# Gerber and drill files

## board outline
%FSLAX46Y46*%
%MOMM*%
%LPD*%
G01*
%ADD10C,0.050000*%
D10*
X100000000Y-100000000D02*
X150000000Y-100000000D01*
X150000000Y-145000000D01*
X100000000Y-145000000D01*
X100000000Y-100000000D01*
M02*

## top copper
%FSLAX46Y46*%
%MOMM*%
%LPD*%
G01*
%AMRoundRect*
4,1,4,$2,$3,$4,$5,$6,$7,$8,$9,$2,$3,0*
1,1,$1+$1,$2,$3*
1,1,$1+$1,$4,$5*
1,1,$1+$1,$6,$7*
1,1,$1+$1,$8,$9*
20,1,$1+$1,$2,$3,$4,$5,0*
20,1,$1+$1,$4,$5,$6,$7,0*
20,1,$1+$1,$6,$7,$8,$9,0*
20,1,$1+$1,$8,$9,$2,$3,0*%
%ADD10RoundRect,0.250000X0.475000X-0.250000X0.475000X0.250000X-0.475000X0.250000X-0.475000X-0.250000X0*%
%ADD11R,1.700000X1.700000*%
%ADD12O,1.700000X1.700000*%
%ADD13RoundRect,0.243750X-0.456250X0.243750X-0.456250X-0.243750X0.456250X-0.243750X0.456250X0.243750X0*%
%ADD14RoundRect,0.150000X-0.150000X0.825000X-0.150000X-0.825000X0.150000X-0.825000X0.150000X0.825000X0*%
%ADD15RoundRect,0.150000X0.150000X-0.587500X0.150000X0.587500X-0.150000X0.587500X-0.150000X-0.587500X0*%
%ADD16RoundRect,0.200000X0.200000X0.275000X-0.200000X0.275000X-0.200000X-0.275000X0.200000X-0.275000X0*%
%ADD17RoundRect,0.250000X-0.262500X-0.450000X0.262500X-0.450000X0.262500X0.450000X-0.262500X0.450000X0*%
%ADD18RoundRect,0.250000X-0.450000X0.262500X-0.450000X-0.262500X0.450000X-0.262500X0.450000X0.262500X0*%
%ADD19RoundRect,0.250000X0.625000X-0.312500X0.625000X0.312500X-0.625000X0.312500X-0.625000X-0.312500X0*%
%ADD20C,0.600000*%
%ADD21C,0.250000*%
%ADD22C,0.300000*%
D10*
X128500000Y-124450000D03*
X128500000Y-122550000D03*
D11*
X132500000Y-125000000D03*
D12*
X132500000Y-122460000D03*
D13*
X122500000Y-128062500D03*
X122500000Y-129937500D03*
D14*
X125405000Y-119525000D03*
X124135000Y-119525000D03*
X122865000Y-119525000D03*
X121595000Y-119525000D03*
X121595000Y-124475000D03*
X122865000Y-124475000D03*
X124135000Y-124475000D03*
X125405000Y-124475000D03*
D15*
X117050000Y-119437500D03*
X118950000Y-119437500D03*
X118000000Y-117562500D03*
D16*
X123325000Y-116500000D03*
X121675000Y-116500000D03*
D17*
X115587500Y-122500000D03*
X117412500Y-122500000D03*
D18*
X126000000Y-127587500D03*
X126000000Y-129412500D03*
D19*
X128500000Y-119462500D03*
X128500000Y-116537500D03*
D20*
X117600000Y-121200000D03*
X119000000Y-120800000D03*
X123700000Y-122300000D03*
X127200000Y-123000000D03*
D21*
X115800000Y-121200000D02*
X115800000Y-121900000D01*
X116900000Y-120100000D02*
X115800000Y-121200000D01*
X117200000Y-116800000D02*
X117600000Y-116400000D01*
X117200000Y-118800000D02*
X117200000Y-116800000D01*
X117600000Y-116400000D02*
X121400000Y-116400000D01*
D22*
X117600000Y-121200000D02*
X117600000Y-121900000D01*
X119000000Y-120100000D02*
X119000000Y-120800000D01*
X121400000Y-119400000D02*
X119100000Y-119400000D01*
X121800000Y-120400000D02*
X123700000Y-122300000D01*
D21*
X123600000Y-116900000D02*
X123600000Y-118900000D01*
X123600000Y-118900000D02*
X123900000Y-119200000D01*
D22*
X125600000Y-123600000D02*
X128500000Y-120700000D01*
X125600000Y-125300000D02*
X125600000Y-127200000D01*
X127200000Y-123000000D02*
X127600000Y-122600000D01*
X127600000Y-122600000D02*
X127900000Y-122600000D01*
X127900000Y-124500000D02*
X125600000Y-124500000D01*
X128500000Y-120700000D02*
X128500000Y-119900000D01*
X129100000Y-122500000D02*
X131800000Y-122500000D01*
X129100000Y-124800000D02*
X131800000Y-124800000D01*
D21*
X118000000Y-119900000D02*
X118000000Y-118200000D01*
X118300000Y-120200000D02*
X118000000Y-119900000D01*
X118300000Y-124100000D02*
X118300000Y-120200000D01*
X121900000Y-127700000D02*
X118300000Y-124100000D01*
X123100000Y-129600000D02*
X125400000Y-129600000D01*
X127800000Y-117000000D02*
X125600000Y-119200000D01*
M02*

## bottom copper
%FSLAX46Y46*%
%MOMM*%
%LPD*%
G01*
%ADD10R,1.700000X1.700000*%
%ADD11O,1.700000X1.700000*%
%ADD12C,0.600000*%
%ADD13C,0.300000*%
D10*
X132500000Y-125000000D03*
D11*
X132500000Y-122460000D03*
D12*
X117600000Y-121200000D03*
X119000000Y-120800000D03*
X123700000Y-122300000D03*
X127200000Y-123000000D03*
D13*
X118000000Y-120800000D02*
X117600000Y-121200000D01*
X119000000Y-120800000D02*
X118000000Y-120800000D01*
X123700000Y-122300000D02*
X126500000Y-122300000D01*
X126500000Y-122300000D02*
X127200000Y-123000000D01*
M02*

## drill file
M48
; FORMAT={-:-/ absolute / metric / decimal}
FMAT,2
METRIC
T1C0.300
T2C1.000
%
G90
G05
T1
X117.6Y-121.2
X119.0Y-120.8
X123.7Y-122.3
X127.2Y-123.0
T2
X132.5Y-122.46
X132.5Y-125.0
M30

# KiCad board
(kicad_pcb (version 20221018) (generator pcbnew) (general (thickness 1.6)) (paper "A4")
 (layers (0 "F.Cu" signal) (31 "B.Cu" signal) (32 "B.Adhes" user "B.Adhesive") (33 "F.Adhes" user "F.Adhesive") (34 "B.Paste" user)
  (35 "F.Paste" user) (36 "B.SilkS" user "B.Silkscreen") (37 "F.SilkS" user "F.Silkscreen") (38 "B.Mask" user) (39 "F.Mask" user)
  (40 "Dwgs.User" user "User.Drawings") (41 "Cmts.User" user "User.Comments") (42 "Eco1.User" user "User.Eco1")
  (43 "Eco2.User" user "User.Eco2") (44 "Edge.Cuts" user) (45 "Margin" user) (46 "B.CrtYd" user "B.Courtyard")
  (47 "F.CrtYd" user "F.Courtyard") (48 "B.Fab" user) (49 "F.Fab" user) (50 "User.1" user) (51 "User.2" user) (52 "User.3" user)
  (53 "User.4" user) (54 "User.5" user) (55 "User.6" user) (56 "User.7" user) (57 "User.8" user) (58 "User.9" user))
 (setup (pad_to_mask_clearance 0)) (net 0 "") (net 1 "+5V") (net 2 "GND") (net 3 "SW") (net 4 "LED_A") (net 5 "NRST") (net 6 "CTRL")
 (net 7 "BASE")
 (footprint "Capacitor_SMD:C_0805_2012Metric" (layer "F.Cu") (at 128.5 123.5 90)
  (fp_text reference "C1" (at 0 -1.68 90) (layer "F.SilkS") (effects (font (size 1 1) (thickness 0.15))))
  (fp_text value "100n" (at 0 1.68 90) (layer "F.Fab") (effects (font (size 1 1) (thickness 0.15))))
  (pad "1" smd roundrect (at -0.95 0 90) (size 1 1.45) (layers "F.Cu" "F.Paste" "F.Mask") (roundrect_rratio 0.25) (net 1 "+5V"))
  (pad "2" smd roundrect (at 0.95 0 90) (size 1 1.45) (layers "F.Cu" "F.Paste" "F.Mask") (roundrect_rratio 0.25) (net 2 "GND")))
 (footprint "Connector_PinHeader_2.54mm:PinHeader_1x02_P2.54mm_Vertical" (layer "F.Cu") (at 132.5 125 180)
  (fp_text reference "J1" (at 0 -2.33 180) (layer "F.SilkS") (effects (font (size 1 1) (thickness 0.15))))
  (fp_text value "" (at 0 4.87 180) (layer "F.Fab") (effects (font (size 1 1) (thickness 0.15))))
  (pad "1" thru_hole rect (at 0 0 180) (size 1.7 1.7) (drill 1) (layers "*.Cu" "*.Mask") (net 1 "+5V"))
  (pad "2" thru_hole oval (at 0 2.54 180) (size 1.7 1.7) (drill 1) (layers "*.Cu" "*.Mask") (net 2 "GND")))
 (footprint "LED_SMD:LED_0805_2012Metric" (layer "F.Cu") (at 122.5 129 -90)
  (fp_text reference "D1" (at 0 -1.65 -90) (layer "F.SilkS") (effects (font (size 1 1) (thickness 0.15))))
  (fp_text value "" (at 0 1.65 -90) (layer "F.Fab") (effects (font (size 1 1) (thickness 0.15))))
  (pad "1" smd roundrect (at -0.9375 0 270) (size 0.975 1.4) (layers "F.Cu" "F.Paste" "F.Mask") (roundrect_rratio 0.25) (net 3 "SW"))
  (pad "2" smd roundrect (at 0.9375 0 270) (size 0.975 1.4) (layers "F.Cu" "F.Paste" "F.Mask") (roundrect_rratio 0.25) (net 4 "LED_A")))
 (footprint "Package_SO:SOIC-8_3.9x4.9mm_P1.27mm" (layer "F.Cu") (at 123.5 122 -90)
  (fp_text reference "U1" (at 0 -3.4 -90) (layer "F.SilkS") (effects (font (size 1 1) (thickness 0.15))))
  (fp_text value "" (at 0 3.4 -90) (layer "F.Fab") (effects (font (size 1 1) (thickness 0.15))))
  (pad "1" smd roundrect (at -2.475 -1.905 270) (size 1.95 0.6) (layers "F.Cu" "F.Paste" "F.Mask") (roundrect_rratio 0.25) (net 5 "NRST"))
  (pad "2" smd roundrect (at -2.475 -0.635 270) (size 1.95 0.6) (layers "F.Cu" "F.Paste" "F.Mask") (roundrect_rratio 0.25) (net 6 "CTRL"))
  (pad "3" smd roundrect (at -2.475 0.635 270) (size 1.95 0.6) (layers "F.Cu" "F.Paste" "F.Mask") (roundrect_rratio 0.25))
  (pad "4" smd roundrect (at -2.475 1.905 270) (size 1.95 0.6) (layers "F.Cu" "F.Paste" "F.Mask") (roundrect_rratio 0.25) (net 2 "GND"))
  (pad "5" smd roundrect (at 2.475 1.905 270) (size 1.95 0.6) (layers "F.Cu" "F.Paste" "F.Mask") (roundrect_rratio 0.25))
  (pad "6" smd roundrect (at 2.475 0.635 270) (size 1.95 0.6) (layers "F.Cu" "F.Paste" "F.Mask") (roundrect_rratio 0.25))
  (pad "7" smd roundrect (at 2.475 -0.635 270) (size 1.95 0.6) (layers "F.Cu" "F.Paste" "F.Mask") (roundrect_rratio 0.25))
  (pad "8" smd roundrect (at 2.475 -1.905 270) (size 1.95 0.6) (layers "F.Cu" "F.Paste" "F.Mask") (roundrect_rratio 0.25) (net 1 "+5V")))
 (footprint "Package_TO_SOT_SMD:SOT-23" (layer "F.Cu") (at 118 118.5 90)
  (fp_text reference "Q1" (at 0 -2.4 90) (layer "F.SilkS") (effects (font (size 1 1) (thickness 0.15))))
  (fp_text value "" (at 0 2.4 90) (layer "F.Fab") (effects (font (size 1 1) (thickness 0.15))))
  (pad "1" smd roundrect (at -0.9375 -0.95 90) (size 1.475 0.6) (layers "F.Cu" "F.Paste" "F.Mask") (roundrect_rratio 0.25) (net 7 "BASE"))
  (pad "2" smd roundrect (at -0.9375 0.95 90) (size 1.475 0.6) (layers "F.Cu" "F.Paste" "F.Mask") (roundrect_rratio 0.25) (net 2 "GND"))
  (pad "3" smd roundrect (at 0.9375 0 90) (size 1.475 0.6) (layers "F.Cu" "F.Paste" "F.Mask") (roundrect_rratio 0.25) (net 3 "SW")))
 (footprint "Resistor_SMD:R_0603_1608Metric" (layer "F.Cu") (at 122.5 116.5 180)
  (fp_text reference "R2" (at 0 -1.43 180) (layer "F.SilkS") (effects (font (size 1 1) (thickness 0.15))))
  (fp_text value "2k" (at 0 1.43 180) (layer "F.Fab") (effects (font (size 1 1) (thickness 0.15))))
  (pad "1" smd roundrect (at -0.825 0 180) (size 0.8 0.95) (layers "F.Cu" "F.Paste" "F.Mask") (roundrect_rratio 0.25) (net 6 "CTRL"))
  (pad "2" smd roundrect (at 0.825 0 180) (size 0.8 0.95) (layers "F.Cu" "F.Paste" "F.Mask") (roundrect_rratio 0.25) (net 7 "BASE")))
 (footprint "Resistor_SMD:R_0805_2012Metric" (layer "F.Cu") (at 116.5 122.5)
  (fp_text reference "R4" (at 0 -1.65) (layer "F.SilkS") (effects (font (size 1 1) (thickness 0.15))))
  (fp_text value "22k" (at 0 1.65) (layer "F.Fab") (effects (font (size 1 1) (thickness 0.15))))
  (pad "1" smd roundrect (at -0.9125 0) (size 1.025 1.4) (layers "F.Cu" "F.Paste" "F.Mask") (roundrect_rratio 0.243902) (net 7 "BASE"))
  (pad "2" smd roundrect (at 0.9125 0) (size 1.025 1.4) (layers "F.Cu" "F.Paste" "F.Mask") (roundrect_rratio 0.243902) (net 2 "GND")))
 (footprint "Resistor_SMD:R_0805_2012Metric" (layer "F.Cu") (at 126 128.5 -90)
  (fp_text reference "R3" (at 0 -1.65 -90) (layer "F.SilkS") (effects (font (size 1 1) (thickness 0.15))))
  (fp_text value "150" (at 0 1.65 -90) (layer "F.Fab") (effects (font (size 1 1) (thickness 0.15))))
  (pad "1" smd roundrect (at -0.9125 0 270) (size 1.025 1.4) (layers "F.Cu" "F.Paste" "F.Mask") (roundrect_rratio 0.243902) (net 1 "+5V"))
  (pad "2" smd roundrect (at 0.9125 0 270) (size 1.025 1.4) (layers "F.Cu" "F.Paste" "F.Mask") (roundrect_rratio 0.243902) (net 4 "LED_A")))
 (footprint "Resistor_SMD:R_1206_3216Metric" (layer "F.Cu") (at 128.5 118 90)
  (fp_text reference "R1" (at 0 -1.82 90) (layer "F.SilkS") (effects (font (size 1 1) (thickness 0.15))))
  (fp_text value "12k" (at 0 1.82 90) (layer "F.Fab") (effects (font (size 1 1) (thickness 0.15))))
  (pad "1" smd roundrect (at -1.4625 0 90) (size 1.125 1.75) (layers "F.Cu" "F.Paste" "F.Mask") (roundrect_rratio 0.222222) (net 1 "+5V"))
  (pad "2" smd roundrect (at 1.4625 0 90) (size 1.125 1.75) (layers "F.Cu" "F.Paste" "F.Mask") (roundrect_rratio 0.222222) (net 5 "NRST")))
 (gr_rect (start 100 100) (end 150 145) (stroke (width 0.05) (type default)) (fill none) (layer "Edge.Cuts"))
 (segment (start 115.8 121.2) (end 115.8 121.9) (width 0.25) (layer "F.Cu") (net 7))
 (segment (start 116.9 120.1) (end 115.8 121.2) (width 0.25) (layer "F.Cu") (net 7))
 (segment (start 117.2 116.8) (end 117.6 116.4) (width 0.25) (layer "F.Cu") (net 7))
 (segment (start 117.2 118.8) (end 117.2 116.8) (width 0.25) (layer "F.Cu") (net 7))
 (segment (start 117.6 116.4) (end 121.4 116.4) (width 0.25) (layer "F.Cu") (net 7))
 (segment (start 117.6 121.2) (end 117.6 121.9) (width 0.3) (layer "F.Cu") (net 2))
 (segment (start 119 120.1) (end 119 120.8) (width 0.3) (layer "F.Cu") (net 2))
 (segment (start 121.4 119.4) (end 119.1 119.4) (width 0.3) (layer "F.Cu") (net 2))
 (segment (start 121.8 120.4) (end 123.7 122.3) (width 0.3) (layer "F.Cu") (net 2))
 (segment (start 123.6 116.9) (end 123.6 118.9) (width 0.25) (layer "F.Cu") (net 6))
 (segment (start 123.6 118.9) (end 123.9 119.2) (width 0.25) (layer "F.Cu") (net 6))
 (segment (start 125.6 123.6) (end 128.5 120.7) (width 0.3) (layer "F.Cu") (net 1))
 (segment (start 125.6 125.3) (end 125.6 127.2) (width 0.3) (layer "F.Cu") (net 1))
 (segment (start 127.2 123) (end 127.6 122.6) (width 0.3) (layer "F.Cu") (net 2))
 (segment (start 127.6 122.6) (end 127.9 122.6) (width 0.3) (layer "F.Cu") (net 2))
 (segment (start 127.9 124.5) (end 125.6 124.5) (width 0.3) (layer "F.Cu") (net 1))
 (segment (start 128.5 120.7) (end 128.5 119.9) (width 0.3) (layer "F.Cu") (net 1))
 (segment (start 129.1 122.5) (end 131.8 122.5) (width 0.3) (layer "F.Cu") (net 2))
 (segment (start 129.1 124.8) (end 131.8 124.8) (width 0.3) (layer "F.Cu") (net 1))
 (via (at 117.6 121.2) (size 0.6) (drill 0.3) (layers "F.Cu" "B.Cu") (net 2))
 (via (at 119 120.8) (size 0.6) (drill 0.3) (layers "F.Cu" "B.Cu") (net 2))
 (via (at 123.7 122.3) (size 0.6) (drill 0.3) (layers "F.Cu" "B.Cu") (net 2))
 (via (at 127.2 123) (size 0.6) (drill 0.3) (layers "F.Cu" "B.Cu") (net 2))
 (segment (start 118 119.9) (end 118 118.2) (width 0.25) (layer "F.Cu") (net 3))
 (segment (start 118 120.8) (end 117.6 121.2) (width 0.3) (layer "B.Cu") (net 2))
 (segment (start 118.3 120.2) (end 118 119.9) (width 0.25) (layer "F.Cu") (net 3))
 (segment (start 118.3 124.1) (end 118.3 120.2) (width 0.25) (layer "F.Cu") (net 3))
 (segment (start 119 120.8) (end 118 120.8) (width 0.3) (layer "B.Cu") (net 2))
 (segment (start 121.9 127.7) (end 118.3 124.1) (width 0.25) (layer "F.Cu") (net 3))
 (segment (start 123.1 129.6) (end 125.4 129.6) (width 0.25) (layer "F.Cu") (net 4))
 (segment (start 123.7 122.3) (end 126.5 122.3) (width 0.3) (layer "B.Cu") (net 2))
 (segment (start 126.5 122.3) (end 127.2 123) (width 0.3) (layer "B.Cu") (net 2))
 (segment (start 127.8 117) (end 125.6 119.2) (width 0.25) (layer "F.Cu") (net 5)))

